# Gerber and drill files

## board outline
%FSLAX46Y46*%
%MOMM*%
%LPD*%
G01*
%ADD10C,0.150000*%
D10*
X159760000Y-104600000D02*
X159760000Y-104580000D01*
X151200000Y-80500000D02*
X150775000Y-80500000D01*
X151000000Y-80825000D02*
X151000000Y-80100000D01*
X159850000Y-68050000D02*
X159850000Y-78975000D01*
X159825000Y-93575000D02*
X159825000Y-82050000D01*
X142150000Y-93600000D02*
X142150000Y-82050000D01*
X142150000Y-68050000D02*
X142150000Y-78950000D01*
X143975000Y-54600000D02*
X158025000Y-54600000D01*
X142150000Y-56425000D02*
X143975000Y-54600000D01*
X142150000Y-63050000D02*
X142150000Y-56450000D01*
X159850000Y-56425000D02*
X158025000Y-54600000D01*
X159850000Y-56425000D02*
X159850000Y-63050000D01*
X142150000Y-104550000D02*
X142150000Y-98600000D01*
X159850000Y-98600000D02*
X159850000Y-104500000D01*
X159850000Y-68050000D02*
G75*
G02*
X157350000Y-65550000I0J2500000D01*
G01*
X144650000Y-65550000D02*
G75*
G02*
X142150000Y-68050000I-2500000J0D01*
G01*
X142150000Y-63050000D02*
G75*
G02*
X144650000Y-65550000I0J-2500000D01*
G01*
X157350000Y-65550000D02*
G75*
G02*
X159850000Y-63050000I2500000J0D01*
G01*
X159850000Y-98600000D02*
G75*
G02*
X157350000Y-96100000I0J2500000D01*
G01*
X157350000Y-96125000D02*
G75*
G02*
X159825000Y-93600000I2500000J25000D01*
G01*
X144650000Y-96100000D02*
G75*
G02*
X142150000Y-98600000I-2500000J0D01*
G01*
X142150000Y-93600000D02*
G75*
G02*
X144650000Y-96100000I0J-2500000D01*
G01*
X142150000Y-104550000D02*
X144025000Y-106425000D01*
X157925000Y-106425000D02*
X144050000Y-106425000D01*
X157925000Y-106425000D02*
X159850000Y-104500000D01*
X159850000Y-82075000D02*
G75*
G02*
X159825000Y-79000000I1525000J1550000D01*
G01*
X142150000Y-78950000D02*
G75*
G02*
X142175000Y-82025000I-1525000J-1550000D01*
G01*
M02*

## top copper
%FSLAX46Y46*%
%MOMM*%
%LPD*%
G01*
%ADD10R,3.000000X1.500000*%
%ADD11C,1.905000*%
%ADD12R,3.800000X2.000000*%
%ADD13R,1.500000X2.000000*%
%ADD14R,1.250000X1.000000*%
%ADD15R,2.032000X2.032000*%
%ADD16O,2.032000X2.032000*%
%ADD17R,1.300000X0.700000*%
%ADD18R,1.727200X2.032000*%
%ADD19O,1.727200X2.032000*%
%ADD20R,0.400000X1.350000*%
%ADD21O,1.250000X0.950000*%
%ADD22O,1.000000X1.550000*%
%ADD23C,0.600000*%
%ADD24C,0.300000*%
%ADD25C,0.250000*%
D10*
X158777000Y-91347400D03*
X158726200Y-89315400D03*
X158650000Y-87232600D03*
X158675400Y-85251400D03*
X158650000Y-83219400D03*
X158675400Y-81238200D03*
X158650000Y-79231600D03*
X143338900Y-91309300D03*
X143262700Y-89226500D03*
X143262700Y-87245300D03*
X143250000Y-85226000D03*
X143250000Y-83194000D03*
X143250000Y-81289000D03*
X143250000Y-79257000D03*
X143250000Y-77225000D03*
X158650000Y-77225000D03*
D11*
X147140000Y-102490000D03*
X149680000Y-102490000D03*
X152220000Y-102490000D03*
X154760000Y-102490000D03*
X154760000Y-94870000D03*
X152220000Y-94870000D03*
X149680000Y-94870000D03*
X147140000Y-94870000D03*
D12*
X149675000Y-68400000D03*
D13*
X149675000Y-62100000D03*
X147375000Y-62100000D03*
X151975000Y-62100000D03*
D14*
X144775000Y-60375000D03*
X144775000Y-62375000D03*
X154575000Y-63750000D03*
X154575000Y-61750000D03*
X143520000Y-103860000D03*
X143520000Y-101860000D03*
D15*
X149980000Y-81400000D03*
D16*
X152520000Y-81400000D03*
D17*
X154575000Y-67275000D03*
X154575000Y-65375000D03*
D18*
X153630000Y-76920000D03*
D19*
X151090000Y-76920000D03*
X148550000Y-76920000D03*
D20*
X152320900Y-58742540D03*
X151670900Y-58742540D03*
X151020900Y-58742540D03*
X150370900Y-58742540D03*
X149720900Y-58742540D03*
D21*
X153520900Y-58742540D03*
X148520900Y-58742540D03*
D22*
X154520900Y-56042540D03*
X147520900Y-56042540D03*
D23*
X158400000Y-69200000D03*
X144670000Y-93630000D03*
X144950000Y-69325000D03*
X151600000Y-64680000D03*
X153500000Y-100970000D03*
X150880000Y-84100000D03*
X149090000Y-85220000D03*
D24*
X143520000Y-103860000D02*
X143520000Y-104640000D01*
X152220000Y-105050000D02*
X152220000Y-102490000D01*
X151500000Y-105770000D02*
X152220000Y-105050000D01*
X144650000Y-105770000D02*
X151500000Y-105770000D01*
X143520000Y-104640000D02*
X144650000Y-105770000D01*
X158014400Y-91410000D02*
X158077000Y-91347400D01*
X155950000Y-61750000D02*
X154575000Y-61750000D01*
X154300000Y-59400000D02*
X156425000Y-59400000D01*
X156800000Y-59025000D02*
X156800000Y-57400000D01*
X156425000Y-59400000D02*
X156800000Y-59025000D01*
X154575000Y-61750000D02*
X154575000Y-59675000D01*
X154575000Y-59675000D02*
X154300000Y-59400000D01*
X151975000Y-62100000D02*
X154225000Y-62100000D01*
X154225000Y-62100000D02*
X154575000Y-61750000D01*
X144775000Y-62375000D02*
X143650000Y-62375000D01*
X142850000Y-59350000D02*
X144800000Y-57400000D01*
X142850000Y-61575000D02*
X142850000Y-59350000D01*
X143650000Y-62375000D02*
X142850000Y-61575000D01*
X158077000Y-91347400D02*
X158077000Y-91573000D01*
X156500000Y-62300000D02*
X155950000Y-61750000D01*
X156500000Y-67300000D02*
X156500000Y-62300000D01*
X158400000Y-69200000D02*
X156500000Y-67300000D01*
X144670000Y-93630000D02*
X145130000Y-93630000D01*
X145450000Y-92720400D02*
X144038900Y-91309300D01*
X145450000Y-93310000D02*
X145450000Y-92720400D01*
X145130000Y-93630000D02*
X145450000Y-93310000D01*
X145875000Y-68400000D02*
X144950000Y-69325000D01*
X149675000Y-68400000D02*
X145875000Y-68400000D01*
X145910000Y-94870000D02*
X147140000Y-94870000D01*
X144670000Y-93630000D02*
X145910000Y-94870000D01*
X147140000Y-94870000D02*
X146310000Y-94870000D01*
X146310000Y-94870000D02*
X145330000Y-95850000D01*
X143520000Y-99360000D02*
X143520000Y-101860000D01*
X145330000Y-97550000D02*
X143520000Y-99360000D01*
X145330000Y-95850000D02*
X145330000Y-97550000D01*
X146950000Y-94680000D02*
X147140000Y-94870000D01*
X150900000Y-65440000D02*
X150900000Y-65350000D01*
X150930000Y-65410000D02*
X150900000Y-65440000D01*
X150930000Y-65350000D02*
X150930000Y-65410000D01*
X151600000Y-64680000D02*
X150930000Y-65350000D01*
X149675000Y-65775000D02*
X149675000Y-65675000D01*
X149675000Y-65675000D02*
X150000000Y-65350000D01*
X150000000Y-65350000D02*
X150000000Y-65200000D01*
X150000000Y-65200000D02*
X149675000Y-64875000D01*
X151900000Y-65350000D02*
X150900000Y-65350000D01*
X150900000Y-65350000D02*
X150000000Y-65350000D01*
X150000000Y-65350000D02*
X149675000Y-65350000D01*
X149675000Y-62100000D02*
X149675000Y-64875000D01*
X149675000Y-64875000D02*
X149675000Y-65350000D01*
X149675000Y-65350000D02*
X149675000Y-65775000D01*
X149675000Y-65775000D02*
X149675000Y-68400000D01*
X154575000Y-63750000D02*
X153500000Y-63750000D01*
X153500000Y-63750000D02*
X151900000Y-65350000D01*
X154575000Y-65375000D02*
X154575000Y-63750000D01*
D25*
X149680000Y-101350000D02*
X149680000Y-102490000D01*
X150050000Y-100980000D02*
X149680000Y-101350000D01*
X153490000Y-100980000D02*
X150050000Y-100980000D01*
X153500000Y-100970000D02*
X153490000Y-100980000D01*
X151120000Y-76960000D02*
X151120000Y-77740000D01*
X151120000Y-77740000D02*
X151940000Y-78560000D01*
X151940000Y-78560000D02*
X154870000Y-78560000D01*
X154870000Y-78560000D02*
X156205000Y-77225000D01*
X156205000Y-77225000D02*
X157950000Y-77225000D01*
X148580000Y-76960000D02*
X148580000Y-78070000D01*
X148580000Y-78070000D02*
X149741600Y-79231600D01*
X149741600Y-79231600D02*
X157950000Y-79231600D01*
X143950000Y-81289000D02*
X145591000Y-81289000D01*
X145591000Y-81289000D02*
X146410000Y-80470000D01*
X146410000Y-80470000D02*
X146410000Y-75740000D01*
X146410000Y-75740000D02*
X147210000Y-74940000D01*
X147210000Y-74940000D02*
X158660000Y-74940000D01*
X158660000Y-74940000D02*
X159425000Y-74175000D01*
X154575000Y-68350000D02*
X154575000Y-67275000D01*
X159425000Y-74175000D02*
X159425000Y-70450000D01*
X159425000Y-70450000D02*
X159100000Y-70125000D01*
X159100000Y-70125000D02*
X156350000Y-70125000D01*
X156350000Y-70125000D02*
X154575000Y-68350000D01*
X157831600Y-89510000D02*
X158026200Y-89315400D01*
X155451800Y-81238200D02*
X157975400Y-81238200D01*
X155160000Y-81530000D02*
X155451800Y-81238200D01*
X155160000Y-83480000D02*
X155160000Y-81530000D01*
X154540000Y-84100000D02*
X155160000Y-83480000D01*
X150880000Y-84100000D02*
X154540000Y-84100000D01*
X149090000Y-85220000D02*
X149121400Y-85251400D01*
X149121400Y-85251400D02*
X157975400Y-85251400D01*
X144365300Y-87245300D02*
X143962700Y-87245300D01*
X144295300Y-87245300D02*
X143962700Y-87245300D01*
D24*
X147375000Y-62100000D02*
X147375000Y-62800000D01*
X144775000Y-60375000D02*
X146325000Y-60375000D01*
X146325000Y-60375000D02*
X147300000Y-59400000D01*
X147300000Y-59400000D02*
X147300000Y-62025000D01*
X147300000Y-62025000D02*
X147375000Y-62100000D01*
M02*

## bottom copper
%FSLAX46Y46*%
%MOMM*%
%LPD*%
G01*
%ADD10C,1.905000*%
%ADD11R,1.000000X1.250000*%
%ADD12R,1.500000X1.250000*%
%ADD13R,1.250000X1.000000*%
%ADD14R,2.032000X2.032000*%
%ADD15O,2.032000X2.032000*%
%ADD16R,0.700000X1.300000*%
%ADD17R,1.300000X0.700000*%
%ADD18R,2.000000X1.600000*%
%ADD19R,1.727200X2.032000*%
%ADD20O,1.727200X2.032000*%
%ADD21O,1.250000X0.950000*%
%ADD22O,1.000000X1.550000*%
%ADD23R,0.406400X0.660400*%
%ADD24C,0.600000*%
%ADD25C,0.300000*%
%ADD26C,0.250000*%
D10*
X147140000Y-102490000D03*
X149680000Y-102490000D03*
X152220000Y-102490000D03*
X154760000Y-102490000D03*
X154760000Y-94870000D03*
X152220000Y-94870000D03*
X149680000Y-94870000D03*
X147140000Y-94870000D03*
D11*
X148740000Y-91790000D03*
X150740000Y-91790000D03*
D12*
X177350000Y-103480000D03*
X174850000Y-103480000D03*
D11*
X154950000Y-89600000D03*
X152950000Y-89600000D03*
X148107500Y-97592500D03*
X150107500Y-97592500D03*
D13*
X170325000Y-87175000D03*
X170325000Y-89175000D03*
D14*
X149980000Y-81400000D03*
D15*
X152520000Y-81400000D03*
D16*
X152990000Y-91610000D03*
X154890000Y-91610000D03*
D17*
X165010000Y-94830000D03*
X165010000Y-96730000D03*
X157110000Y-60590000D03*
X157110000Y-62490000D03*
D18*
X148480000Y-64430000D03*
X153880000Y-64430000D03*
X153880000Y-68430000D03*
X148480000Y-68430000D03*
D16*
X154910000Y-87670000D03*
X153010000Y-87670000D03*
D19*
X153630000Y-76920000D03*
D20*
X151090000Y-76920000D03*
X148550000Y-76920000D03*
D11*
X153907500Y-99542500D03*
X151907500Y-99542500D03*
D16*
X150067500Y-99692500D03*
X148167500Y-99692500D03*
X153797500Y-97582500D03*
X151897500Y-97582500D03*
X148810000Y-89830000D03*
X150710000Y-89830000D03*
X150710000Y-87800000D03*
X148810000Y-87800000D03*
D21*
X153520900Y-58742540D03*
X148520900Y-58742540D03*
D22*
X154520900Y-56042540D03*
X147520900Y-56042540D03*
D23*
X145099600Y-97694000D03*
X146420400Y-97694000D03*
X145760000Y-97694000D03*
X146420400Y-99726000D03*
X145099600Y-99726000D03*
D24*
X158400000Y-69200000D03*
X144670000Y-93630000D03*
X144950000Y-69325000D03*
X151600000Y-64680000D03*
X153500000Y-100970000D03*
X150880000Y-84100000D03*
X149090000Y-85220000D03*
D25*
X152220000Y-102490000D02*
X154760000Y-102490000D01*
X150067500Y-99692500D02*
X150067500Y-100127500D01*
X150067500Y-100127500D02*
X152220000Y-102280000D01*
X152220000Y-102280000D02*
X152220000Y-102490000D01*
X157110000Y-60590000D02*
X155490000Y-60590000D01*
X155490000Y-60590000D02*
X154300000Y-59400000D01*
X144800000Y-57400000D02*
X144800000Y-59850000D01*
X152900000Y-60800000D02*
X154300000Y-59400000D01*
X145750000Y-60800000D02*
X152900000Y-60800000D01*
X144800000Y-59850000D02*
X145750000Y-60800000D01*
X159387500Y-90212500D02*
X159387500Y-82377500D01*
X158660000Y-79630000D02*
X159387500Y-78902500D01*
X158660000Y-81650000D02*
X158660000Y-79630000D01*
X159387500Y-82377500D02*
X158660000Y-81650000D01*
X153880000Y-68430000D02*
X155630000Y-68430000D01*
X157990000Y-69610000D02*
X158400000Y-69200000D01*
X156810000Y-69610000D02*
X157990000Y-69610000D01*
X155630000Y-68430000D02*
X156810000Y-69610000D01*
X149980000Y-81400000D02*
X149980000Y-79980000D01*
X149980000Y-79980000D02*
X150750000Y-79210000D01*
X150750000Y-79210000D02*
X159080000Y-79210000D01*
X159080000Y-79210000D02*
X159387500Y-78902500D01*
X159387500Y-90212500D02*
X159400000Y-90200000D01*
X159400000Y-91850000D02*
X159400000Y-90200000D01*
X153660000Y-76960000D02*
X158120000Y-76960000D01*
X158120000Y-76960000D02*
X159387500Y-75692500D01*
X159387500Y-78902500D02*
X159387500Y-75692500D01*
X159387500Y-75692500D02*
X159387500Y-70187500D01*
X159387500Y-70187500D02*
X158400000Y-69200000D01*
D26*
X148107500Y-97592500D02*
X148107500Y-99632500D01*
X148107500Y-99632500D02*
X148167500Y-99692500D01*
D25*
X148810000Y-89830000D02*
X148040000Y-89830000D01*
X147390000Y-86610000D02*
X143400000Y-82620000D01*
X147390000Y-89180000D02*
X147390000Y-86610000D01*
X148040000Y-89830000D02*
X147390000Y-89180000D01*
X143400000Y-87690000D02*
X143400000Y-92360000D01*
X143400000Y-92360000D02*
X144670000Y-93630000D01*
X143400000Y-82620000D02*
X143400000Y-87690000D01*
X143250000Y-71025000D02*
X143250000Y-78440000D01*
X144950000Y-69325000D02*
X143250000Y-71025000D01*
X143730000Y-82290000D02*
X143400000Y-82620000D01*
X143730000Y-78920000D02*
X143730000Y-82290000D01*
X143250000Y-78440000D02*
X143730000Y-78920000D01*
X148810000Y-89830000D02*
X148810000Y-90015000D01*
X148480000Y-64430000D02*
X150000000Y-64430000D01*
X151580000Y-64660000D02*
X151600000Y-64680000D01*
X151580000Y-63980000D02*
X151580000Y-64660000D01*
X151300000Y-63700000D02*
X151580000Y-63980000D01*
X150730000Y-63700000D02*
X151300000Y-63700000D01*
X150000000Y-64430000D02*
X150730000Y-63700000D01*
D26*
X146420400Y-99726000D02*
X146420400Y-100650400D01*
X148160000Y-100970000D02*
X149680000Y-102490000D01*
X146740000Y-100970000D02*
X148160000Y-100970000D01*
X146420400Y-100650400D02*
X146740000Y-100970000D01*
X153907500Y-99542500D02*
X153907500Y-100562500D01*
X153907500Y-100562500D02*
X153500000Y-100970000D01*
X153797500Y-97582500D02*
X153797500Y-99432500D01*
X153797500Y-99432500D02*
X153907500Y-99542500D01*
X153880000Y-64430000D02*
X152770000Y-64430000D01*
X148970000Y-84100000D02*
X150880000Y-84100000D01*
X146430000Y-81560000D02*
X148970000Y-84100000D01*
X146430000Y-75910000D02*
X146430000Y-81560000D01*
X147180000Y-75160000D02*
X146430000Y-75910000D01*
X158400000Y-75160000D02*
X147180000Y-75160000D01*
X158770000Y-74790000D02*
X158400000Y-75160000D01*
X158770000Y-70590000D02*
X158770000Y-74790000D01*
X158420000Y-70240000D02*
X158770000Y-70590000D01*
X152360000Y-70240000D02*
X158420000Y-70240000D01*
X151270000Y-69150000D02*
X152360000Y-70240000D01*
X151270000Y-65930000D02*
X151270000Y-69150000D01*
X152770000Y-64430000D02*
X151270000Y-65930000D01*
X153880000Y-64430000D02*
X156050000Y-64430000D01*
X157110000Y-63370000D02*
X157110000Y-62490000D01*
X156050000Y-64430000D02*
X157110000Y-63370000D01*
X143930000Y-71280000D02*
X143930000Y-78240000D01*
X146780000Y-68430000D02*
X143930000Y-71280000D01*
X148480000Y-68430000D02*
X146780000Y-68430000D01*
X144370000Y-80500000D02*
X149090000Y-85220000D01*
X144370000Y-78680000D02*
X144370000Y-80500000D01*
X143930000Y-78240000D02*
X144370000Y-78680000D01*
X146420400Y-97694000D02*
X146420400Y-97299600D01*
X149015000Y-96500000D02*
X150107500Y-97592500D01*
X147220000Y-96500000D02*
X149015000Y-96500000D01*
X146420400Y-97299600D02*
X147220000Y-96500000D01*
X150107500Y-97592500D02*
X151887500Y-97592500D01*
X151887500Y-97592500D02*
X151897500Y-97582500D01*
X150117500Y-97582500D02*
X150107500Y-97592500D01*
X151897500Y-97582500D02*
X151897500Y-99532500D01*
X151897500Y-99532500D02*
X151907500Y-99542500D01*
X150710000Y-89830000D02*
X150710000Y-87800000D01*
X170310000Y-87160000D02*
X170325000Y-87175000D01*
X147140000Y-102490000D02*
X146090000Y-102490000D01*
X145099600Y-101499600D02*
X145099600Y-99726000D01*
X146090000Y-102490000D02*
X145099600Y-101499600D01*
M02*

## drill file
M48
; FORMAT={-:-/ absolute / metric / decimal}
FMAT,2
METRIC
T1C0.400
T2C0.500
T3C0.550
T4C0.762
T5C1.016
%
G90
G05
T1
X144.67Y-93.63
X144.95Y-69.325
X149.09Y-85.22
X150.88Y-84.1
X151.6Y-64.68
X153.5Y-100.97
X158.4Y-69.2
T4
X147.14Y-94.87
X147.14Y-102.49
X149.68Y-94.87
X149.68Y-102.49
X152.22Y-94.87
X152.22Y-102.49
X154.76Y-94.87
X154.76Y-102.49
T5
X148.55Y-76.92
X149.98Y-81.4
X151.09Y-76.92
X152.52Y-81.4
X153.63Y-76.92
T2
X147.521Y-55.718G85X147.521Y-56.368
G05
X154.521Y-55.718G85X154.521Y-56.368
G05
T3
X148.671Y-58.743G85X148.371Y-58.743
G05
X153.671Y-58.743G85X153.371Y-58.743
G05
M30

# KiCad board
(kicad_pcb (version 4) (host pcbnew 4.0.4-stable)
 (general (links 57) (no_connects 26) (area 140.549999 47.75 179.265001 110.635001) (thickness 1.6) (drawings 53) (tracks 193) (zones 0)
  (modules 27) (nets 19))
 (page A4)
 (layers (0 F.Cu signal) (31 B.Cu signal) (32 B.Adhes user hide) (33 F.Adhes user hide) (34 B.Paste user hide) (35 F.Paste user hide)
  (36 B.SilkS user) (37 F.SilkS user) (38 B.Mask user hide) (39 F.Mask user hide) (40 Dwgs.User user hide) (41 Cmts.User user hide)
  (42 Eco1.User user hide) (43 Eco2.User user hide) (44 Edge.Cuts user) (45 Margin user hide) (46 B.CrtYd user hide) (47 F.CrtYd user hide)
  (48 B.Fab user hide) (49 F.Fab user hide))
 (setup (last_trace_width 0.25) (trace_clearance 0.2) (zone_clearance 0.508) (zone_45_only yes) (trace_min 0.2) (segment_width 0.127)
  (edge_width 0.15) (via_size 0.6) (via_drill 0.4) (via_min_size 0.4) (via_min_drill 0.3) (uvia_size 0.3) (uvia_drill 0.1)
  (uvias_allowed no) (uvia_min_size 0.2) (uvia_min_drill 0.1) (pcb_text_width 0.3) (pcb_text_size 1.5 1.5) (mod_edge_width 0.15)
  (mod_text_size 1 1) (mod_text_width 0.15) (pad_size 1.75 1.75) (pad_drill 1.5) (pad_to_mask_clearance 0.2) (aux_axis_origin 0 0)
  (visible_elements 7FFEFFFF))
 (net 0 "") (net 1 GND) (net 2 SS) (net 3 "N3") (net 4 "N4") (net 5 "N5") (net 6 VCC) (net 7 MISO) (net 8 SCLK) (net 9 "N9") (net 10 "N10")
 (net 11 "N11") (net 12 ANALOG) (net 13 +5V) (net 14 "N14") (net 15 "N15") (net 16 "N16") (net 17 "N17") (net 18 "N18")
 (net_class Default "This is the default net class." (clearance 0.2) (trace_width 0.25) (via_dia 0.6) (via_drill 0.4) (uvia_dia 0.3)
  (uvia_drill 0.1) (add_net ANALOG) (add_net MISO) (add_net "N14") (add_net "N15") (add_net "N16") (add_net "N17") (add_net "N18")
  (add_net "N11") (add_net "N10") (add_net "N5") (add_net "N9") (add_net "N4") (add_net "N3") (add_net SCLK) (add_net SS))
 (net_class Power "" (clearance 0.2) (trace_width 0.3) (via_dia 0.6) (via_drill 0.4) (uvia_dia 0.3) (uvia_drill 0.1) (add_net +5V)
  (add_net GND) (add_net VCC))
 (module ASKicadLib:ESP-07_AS (layer F.Cu) (at 143.95 77.225)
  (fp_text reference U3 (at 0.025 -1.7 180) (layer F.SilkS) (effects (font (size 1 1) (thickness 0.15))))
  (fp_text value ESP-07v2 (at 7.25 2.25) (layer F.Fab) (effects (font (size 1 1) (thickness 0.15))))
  (pad 9 smd rect (at 14.127 14.1224) (size 3 1.5) (drill (offset 0.7 0)) (layers F.Cu F.Paste F.Mask) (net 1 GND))
  (pad 10 smd rect (at 14.0762 12.0904) (size 3 1.5) (drill (offset 0.7 0)) (layers F.Cu F.Paste F.Mask) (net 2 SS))
  (pad 11 smd rect (at 14 10.0076) (size 3 1.5) (drill (offset 0.7 0)) (layers F.Cu F.Paste F.Mask))
  (pad 12 smd rect (at 14.0254 8.0264) (size 3 1.5) (drill (offset 0.7 0)) (layers F.Cu F.Paste F.Mask) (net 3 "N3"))
  (pad 13 smd rect (at 14 5.9944) (size 3 1.5) (drill (offset 0.7 0)) (layers F.Cu F.Paste F.Mask))
  (pad 14 smd rect (at 14.0254 4.0132) (size 3 1.5) (drill (offset 0.7 0)) (layers F.Cu F.Paste F.Mask) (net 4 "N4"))
  (pad 15 smd rect (at 14 2.0066) (size 3 1.5) (drill (offset 0.7 0)) (layers F.Cu F.Paste F.Mask) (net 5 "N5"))
  (pad 8 smd rect (at 0.0889 14.0843) (size 3 1.5) (drill (offset -0.7 0)) (layers F.Cu F.Paste F.Mask) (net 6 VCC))
  (pad 7 smd rect (at 0.0127 12.0015) (size 3 1.5) (drill (offset -0.7 0)) (layers F.Cu F.Paste F.Mask))
  (pad 6 smd rect (at 0.0127 10.0203) (size 3 1.5) (drill (offset -0.7 0)) (layers F.Cu F.Paste F.Mask) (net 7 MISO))
  (pad 5 smd rect (at 0 8.001) (size 3 1.5) (drill (offset -0.7 0)) (layers F.Cu F.Paste F.Mask) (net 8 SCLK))
  (pad 4 smd rect (at 0 5.969) (size 3 1.5) (drill (offset -0.7 0)) (layers F.Cu F.Paste F.Mask))
  (pad 3 smd rect (at 0 4.064) (size 3 1.5) (drill (offset -0.7 0)) (layers F.Cu F.Paste F.Mask) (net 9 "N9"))
  (pad 2 smd rect (at 0 2.032) (size 3 1.5) (drill (offset -0.7 0)) (layers F.Cu F.Paste F.Mask))
  (pad 1 smd rect (at 0 0) (size 3 1.5) (drill (offset -0.7 0)) (layers F.Cu F.Paste F.Mask))
  (pad 16 smd rect (at 14 0) (size 3 1.5) (drill (offset 0.7 0)) (layers F.Cu F.Paste F.Mask) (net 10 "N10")))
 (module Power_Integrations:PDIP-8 (layer F.Cu) (at 150.95 98.68)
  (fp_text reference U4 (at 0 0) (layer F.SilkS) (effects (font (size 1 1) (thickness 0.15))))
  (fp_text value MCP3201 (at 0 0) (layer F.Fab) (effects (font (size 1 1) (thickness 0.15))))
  (pad 1 thru_hole circle (at -3.81 3.81) (size 1.905 1.905) (drill 0.762) (layers *.Cu *.Mask) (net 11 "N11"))
  (pad 2 thru_hole circle (at -1.27 3.81) (size 1.905 1.905) (drill 0.762) (layers *.Cu *.Mask) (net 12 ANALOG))
  (pad 3 thru_hole circle (at 1.27 3.81) (size 1.905 1.905) (drill 0.762) (layers *.Cu *.Mask) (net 1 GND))
  (pad 4 thru_hole circle (at 3.81 3.81) (size 1.905 1.905) (drill 0.762) (layers *.Cu *.Mask) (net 1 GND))
  (pad 5 thru_hole circle (at 3.81 -3.81) (size 1.905 1.905) (drill 0.762) (layers *.Cu *.Mask) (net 2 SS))
  (pad 6 thru_hole circle (at 1.27 -3.81) (size 1.905 1.905) (drill 0.762) (layers *.Cu *.Mask) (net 7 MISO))
  (pad 7 thru_hole circle (at -1.27 -3.81) (size 1.905 1.905) (drill 0.762) (layers *.Cu *.Mask) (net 8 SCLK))
  (pad 8 thru_hole circle (at -3.81 -3.81) (size 1.905 1.905) (drill 0.762) (layers *.Cu *.Mask) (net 6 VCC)))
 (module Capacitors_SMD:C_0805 (layer B.Cu) (at 149.74 91.79)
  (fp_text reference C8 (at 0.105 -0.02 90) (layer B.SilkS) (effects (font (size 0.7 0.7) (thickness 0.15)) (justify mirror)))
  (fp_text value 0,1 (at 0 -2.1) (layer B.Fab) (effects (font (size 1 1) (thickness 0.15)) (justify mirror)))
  (pad 1 smd rect (at -1 0) (size 1 1.25) (layers B.Cu B.Paste B.Mask) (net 1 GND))
  (pad 2 smd rect (at 1 0) (size 1 1.25) (layers B.Cu B.Paste B.Mask) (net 11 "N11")))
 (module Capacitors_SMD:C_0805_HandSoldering (layer B.Cu) (at 176.1 103.48 180)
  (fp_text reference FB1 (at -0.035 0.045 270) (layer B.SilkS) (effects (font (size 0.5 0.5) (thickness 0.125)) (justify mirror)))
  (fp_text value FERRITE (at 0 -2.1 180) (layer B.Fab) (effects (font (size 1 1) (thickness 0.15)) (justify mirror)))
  (pad 1 smd rect (at -1.25 0 180) (size 1.5 1.25) (layers B.Cu B.Paste B.Mask) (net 11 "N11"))
  (pad 2 smd rect (at 1.25 0 180) (size 1.5 1.25) (layers B.Cu B.Paste B.Mask) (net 6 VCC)))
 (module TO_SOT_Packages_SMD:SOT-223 (layer F.Cu) (at 149.675 65.25 270)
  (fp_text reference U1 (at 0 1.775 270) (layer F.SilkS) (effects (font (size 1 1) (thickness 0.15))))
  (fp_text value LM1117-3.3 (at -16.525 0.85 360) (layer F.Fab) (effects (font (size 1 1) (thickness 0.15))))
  (pad 4 smd rect (at 3.15 0 270) (size 2 3.8) (layers F.Cu F.Paste F.Mask) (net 6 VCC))
  (pad 2 smd rect (at -3.15 0 270) (size 2 1.5) (layers F.Cu F.Paste F.Mask) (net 6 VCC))
  (pad 3 smd rect (at -3.15 2.3 270) (size 2 1.5) (layers F.Cu F.Paste F.Mask) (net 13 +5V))
  (pad 1 smd rect (at -3.15 -2.3 270) (size 2 1.5) (layers F.Cu F.Paste F.Mask) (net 1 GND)))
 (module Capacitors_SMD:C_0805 (layer F.Cu) (at 144.775 61.375 270)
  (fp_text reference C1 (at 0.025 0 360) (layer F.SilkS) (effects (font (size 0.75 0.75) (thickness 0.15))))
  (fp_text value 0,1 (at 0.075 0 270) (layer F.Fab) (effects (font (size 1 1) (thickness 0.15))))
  (pad 1 smd rect (at -1 0 270) (size 1 1.25) (layers F.Cu F.Paste F.Mask) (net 13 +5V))
  (pad 2 smd rect (at 1 0 270) (size 1 1.25) (layers F.Cu F.Paste F.Mask) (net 1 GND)))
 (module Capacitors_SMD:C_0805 (layer B.Cu) (at 153.95 89.6 180)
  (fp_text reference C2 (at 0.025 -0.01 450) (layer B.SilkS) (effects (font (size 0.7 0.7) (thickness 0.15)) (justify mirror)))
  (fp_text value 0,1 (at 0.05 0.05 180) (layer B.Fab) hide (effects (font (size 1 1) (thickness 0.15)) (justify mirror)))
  (pad 1 smd rect (at -1 0 180) (size 1 1.25) (layers B.Cu B.Paste B.Mask) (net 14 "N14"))
  (pad 2 smd rect (at 1 0 180) (size 1 1.25) (layers B.Cu B.Paste B.Mask) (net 1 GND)))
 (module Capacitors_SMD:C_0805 (layer B.Cu) (at 149.1075 97.5925)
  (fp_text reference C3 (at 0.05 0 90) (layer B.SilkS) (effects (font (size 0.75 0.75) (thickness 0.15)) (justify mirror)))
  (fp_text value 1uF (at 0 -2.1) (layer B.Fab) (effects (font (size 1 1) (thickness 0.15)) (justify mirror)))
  (pad 1 smd rect (at -1 0) (size 1 1.25) (layers B.Cu B.Paste B.Mask) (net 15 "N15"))
  (pad 2 smd rect (at 1 0) (size 1 1.25) (layers B.Cu B.Paste B.Mask) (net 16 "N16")))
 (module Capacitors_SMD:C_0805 (layer F.Cu) (at 154.575 62.75 90)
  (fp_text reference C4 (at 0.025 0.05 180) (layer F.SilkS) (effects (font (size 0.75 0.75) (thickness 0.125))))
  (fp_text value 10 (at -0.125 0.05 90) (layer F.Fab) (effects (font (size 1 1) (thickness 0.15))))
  (pad 1 smd rect (at -1 0 90) (size 1 1.25) (layers F.Cu F.Paste F.Mask) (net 6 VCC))
  (pad 2 smd rect (at 1 0 90) (size 1 1.25) (layers F.Cu F.Paste F.Mask) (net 1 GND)))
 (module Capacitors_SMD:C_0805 (layer B.Cu) (at 170.325 88.175 270)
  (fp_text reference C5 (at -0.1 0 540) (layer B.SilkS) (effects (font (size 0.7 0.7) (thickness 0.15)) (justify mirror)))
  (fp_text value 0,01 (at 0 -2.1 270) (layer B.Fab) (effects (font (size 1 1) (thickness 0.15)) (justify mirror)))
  (pad 1 smd rect (at -1 0 270) (size 1 1.25) (layers B.Cu B.Paste B.Mask) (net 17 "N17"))
  (pad 2 smd rect (at 1 0 270) (size 1 1.25) (layers B.Cu B.Paste B.Mask) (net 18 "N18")))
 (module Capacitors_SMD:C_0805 (layer F.Cu) (at 143.52 102.86 90)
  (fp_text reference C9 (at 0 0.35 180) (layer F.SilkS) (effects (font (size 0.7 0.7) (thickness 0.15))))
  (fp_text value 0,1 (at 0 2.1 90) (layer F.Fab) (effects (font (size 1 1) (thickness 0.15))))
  (pad 1 smd rect (at -1 0 90) (size 1 1.25) (layers F.Cu F.Paste F.Mask) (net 1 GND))
  (pad 2 smd rect (at 1 0 90) (size 1 1.25) (layers F.Cu F.Paste F.Mask) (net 6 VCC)))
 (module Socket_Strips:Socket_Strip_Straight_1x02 (layer F.Cu) (at 149.98 81.4)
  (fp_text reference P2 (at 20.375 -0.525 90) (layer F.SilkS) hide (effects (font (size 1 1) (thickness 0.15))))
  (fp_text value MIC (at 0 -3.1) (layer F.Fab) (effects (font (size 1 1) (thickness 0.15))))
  (pad 1 thru_hole rect (at 0 0) (size 2.032 2.032) (drill 1.016) (layers *.Cu *.Mask) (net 1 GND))
  (pad 2 thru_hole oval (at 2.54 0) (size 2.032 2.032) (drill 1.016) (layers *.Cu *.Mask) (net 18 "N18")))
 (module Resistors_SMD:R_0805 (layer B.Cu) (at 153.94 91.61)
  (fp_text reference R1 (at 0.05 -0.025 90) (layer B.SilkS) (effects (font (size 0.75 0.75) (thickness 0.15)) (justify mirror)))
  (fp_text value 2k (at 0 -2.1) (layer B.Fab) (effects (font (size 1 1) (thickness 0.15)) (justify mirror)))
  (pad 1 smd rect (at -0.95 0) (size 0.7 1.3) (layers B.Cu B.Paste B.Mask) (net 6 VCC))
  (pad 2 smd rect (at 0.95 0) (size 0.7 1.3) (layers B.Cu B.Paste B.Mask) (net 14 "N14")))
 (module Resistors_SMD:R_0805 (layer F.Cu) (at 154.575 66.325 90)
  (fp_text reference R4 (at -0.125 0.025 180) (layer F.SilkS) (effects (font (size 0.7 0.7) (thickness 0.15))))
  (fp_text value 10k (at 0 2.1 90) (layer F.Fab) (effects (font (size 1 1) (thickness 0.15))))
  (pad 1 smd rect (at -0.95 0 90) (size 0.7 1.3) (layers F.Cu F.Paste F.Mask) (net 9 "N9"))
  (pad 2 smd rect (at 0.95 0 90) (size 0.7 1.3) (layers F.Cu F.Paste F.Mask) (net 6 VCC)))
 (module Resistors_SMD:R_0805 (layer B.Cu) (at 165.01 95.78 270)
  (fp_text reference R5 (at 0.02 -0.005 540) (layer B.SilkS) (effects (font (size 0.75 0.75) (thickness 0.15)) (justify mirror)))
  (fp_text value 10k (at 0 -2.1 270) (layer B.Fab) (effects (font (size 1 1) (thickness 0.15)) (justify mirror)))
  (pad 1 smd rect (at -0.95 0 270) (size 0.7 1.3) (layers B.Cu B.Paste B.Mask) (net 2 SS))
  (pad 2 smd rect (at 0.95 0 270) (size 0.7 1.3) (layers B.Cu B.Paste B.Mask) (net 1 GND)))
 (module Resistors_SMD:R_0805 (layer B.Cu) (at 157.11 61.54 270)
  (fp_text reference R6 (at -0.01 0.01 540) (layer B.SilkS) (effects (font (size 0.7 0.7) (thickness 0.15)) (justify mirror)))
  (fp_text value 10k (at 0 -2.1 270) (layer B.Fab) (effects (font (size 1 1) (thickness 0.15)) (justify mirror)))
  (pad 1 smd rect (at -0.95 0 270) (size 0.7 1.3) (layers B.Cu B.Paste B.Mask) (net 1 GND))
  (pad 2 smd rect (at 0.95 0 270) (size 0.7 1.3) (layers B.Cu B.Paste B.Mask) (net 4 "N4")))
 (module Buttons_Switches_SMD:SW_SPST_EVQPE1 (layer B.Cu) (at 151.18 64.43 180)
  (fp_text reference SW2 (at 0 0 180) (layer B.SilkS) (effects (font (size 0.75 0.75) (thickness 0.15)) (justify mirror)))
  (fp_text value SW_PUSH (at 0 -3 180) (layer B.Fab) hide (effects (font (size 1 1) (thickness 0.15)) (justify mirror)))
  (pad 2 smd rect (at 2.7 0 180) (size 2 1.6) (layers B.Cu B.Paste B.Mask) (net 6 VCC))
  (pad 1 smd rect (at -2.7 0 180) (size 2 1.6) (layers B.Cu B.Paste B.Mask) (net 4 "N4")))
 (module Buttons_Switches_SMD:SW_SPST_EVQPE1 (layer B.Cu) (at 151.18 68.43)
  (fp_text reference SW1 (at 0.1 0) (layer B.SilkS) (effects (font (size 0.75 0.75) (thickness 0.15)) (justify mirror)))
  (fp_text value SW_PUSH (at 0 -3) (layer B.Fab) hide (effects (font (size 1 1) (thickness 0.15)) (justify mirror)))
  (pad 2 smd rect (at 2.7 0) (size 2 1.6) (layers B.Cu B.Paste B.Mask) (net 1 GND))
  (pad 1 smd rect (at -2.7 0) (size 2 1.6) (layers B.Cu B.Paste B.Mask) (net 3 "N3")))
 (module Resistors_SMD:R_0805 (layer B.Cu) (at 153.96 87.67 180)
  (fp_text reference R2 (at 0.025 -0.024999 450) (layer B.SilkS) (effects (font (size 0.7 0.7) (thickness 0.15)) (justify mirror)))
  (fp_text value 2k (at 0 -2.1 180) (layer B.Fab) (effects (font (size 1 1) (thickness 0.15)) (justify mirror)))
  (pad 1 smd rect (at -0.95 0 180) (size 0.7 1.3) (layers B.Cu B.Paste B.Mask) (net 14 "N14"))
  (pad 2 smd rect (at 0.95 0 180) (size 0.7 1.3) (layers B.Cu B.Paste B.Mask) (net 18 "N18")))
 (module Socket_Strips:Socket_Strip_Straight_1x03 (layer F.Cu) (at 153.63 76.92 180)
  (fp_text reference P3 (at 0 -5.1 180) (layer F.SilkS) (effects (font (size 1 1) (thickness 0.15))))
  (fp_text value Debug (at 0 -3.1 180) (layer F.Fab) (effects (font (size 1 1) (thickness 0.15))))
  (pad 1 thru_hole rect (at 0 0 180) (size 1.7272 2.032) (drill 1.016) (layers *.Cu *.Mask) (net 1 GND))
  (pad 2 thru_hole oval (at 2.54 0 180) (size 1.7272 2.032) (drill 1.016) (layers *.Cu *.Mask) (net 10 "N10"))
  (pad 3 thru_hole oval (at 5.08 0 180) (size 1.7272 2.032) (drill 1.016) (layers *.Cu *.Mask) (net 5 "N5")))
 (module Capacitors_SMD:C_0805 (layer B.Cu) (at 152.9075 99.5425 180)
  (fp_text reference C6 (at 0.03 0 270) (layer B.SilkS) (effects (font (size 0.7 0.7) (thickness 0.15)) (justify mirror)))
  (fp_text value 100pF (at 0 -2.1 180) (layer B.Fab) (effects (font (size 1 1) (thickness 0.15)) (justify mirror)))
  (pad 1 smd rect (at -1 0 180) (size 1 1.25) (layers B.Cu B.Paste B.Mask) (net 12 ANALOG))
  (pad 2 smd rect (at 1 0 180) (size 1 1.25) (layers B.Cu B.Paste B.Mask) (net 16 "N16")))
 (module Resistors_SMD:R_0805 (layer B.Cu) (at 149.1175 99.6925 180)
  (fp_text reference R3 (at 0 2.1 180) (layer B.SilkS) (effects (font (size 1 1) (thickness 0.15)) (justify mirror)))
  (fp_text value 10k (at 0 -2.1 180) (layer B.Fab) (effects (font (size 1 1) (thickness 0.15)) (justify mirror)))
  (pad 1 smd rect (at -0.95 0 180) (size 0.7 1.3) (layers B.Cu B.Paste B.Mask) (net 1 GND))
  (pad 2 smd rect (at 0.95 0 180) (size 0.7 1.3) (layers B.Cu B.Paste B.Mask) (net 15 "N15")))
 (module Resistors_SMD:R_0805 (layer B.Cu) (at 152.8475 97.5825 180)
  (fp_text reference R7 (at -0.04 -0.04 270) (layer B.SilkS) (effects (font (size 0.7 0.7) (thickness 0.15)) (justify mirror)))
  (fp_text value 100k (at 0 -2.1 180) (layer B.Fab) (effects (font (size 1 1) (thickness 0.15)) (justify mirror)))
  (pad 1 smd rect (at -0.95 0 180) (size 0.7 1.3) (layers B.Cu B.Paste B.Mask) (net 12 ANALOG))
  (pad 2 smd rect (at 0.95 0 180) (size 0.7 1.3) (layers B.Cu B.Paste B.Mask) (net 16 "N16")))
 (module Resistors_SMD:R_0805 (layer B.Cu) (at 149.76 89.83)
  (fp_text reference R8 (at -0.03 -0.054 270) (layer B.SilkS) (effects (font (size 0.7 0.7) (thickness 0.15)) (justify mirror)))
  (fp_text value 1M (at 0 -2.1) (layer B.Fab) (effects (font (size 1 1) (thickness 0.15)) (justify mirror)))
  (pad 1 smd rect (at -0.95 0) (size 0.7 1.3) (layers B.Cu B.Paste B.Mask) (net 6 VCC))
  (pad 2 smd rect (at 0.95 0) (size 0.7 1.3) (layers B.Cu B.Paste B.Mask) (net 17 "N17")))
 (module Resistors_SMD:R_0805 (layer B.Cu) (at 149.76 87.8 180)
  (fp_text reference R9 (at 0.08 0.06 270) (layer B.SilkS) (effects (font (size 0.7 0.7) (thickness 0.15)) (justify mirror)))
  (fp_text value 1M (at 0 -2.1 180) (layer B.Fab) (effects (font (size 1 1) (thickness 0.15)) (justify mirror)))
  (pad 1 smd rect (at -0.95 0 180) (size 0.7 1.3) (layers B.Cu B.Paste B.Mask) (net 17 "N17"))
  (pad 2 smd rect (at 0.95 0 180) (size 0.7 1.3) (layers B.Cu B.Paste B.Mask) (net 1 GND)))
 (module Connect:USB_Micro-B (layer F.Cu) (at 151.02 57.18 180)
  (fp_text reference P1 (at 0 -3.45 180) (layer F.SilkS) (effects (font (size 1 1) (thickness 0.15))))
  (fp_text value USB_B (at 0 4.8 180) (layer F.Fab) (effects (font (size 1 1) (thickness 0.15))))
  (pad 1 smd rect (at -1.3009 -1.56254 270) (size 1.35 0.4) (layers F.Cu F.Paste F.Mask) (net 13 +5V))
  (pad 2 smd rect (at -0.6509 -1.56254 270) (size 1.35 0.4) (layers F.Cu F.Paste F.Mask))
  (pad 3 smd rect (at -0.0009 -1.56254 270) (size 1.35 0.4) (layers F.Cu F.Paste F.Mask))
  (pad 4 smd rect (at 0.6491 -1.56254 270) (size 1.35 0.4) (layers F.Cu F.Paste F.Mask) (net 1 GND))
  (pad 5 smd rect (at 1.2991 -1.56254 270) (size 1.35 0.4) (layers F.Cu F.Paste F.Mask) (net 1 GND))
  (pad 6 thru_hole oval (at -2.5009 -1.56254 270) (size 0.95 1.25) (drill oval 0.55 0.85) (layers *.Cu *.Mask))
  (pad 6 thru_hole oval (at 2.4991 -1.56254 270) (size 0.95 1.25) (drill oval 0.55 0.85) (layers *.Cu *.Mask))
  (pad 6 thru_hole oval (at -3.5009 1.13746 270) (size 1.55 1) (drill oval 1.15 0.5) (layers *.Cu *.Mask))
  (pad 6 thru_hole oval (at 3.4991 1.13746 270) (size 1.55 1) (drill oval 1.15 0.5) (layers *.Cu *.Mask)))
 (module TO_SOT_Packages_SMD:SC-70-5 (layer B.Cu) (at 145.76 98.71)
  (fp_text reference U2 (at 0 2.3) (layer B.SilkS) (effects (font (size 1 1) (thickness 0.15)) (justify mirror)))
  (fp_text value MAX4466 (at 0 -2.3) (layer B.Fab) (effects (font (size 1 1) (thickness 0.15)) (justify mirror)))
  (pad 1 smd rect (at -0.6604 -1.016) (size 0.4064 0.6604) (layers B.Cu B.Paste B.Mask) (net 17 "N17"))
  (pad 3 smd rect (at 0.6604 -1.016) (size 0.4064 0.6604) (layers B.Cu B.Paste B.Mask) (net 16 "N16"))
  (pad 2 smd rect (at 0 -1.016) (size 0.4064 0.6604) (layers B.Cu B.Paste B.Mask) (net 1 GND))
  (pad 4 smd rect (at 0.6604 1.016) (size 0.4064 0.6604) (layers B.Cu B.Paste B.Mask) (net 12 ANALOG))
  (pad 5 smd rect (at -0.6604 1.016) (size 0.4064 0.6604) (layers B.Cu B.Paste B.Mask) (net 11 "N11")))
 (gr_line (start 159.76 104.6) (end 159.76 104.58) (angle 90) (layer Edge.Cuts) (width 0.15))
 (gr_line (start 151.2 80.5) (end 150.775 80.5) (angle 90) (layer Edge.Cuts) (width 0.15))
 (gr_line (start 151 80.825) (end 151 80.1) (angle 90) (layer Edge.Cuts) (width 0.15))
 (gr_line (start 159.85 68.05) (end 159.85 78.975) (angle 90) (layer Edge.Cuts) (width 0.15))
 (gr_line (start 159.825 93.575) (end 159.825 82.05) (angle 90) (layer Edge.Cuts) (width 0.15))
 (gr_line (start 142.15 93.6) (end 142.15 82.05) (angle 90) (layer Edge.Cuts) (width 0.15))
 (gr_line (start 142.15 68.05) (end 142.15 78.95) (angle 90) (layer Edge.Cuts) (width 0.15))
 (gr_line (start 143.975 54.6) (end 158.025 54.6) (angle 90) (layer Edge.Cuts) (width 0.15))
 (gr_line (start 142.15 56.425) (end 143.975 54.6) (angle 90) (layer Edge.Cuts) (width 0.15))
 (gr_line (start 142.15 63.05) (end 142.15 56.45) (angle 90) (layer Edge.Cuts) (width 0.15))
 (gr_line (start 159.85 56.425) (end 158.025 54.6) (angle 90) (layer Edge.Cuts) (width 0.15))
 (gr_line (start 159.85 56.425) (end 159.85 63.05) (angle 90) (layer Edge.Cuts) (width 0.15))
 (gr_line (start 142.15 104.55) (end 142.15 98.6) (angle 90) (layer Edge.Cuts) (width 0.15))
 (gr_line (start 159.85 98.6) (end 159.85 104.5) (angle 90) (layer Edge.Cuts) (width 0.15))
 (gr_arc (start 159.85 65.55) (end 159.85 68.05) (angle 90) (layer Edge.Cuts) (width 0.15))
 (gr_arc (start 142.15 65.55) (end 144.65 65.55) (angle 90) (layer Edge.Cuts) (width 0.15))
 (gr_arc (start 142.15 65.55) (end 142.15 63.05) (angle 90) (layer Edge.Cuts) (width 0.15))
 (gr_arc (start 159.85 65.55) (end 157.35 65.55) (angle 90) (layer Edge.Cuts) (width 0.15))
 (gr_arc (start 159.85 96.1) (end 159.85 98.6) (angle 90) (layer Edge.Cuts) (width 0.15))
 (gr_arc (start 159.85 96.1) (end 157.35 96.125) (angle 90) (layer Edge.Cuts) (width 0.15))
 (gr_arc (start 142.15 96.1) (end 144.65 96.1) (angle 90) (layer Edge.Cuts) (width 0.15))
 (gr_arc (start 142.15 96.1) (end 142.15 93.6) (angle 90) (layer Edge.Cuts) (width 0.15))
 (gr_line (start 142.15 104.55) (end 144.025 106.425) (angle 90) (layer Edge.Cuts) (width 0.15))
 (gr_line (start 157.925 106.425) (end 144.05 106.425) (angle 90) (layer Edge.Cuts) (width 0.15))
 (gr_line (start 157.925 106.425) (end 159.85 104.5) (angle 90) (layer Edge.Cuts) (width 0.15))
 (gr_arc (start 161.375 80.525) (end 159.85 82.075) (angle 90) (layer Edge.Cuts) (width 0.15))
 (gr_arc (start 140.625 80.5) (end 142.15 78.95) (angle 90) (layer Edge.Cuts) (width 0.15))
 (segment (start 143.52 103.86) (end 143.52 104.64) (width 0.3) (layer F.Cu) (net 1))
 (segment (start 152.22 105.05) (end 152.22 102.49) (width 0.3) (layer F.Cu) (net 1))
 (segment (start 151.5 105.77) (end 152.22 105.05) (width 0.3) (layer F.Cu) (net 1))
 (segment (start 144.65 105.77) (end 151.5 105.77) (width 0.3) (layer F.Cu) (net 1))
 (segment (start 143.52 104.64) (end 144.65 105.77) (width 0.3) (layer F.Cu) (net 1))
 (segment (start 152.22 102.49) (end 154.76 102.49) (width 0.3) (layer B.Cu) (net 1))
 (segment (start 150.0675 99.6925) (end 150.0675 100.1275) (width 0.3) (layer B.Cu) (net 1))
 (segment (start 150.0675 100.1275) (end 152.22 102.28) (width 0.3) (layer B.Cu) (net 1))
 (segment (start 152.22 102.28) (end 152.22 102.49) (width 0.3) (layer B.Cu) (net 1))
 (segment (start 157.11 60.59) (end 155.49 60.59) (width 0.3) (layer B.Cu) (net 1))
 (segment (start 155.49 60.59) (end 154.3 59.4) (width 0.3) (layer B.Cu) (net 1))
 (segment (start 144.8 57.4) (end 144.8 59.85) (width 0.3) (layer B.Cu) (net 1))
 (segment (start 152.9 60.8) (end 154.3 59.4) (width 0.3) (layer B.Cu) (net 1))
 (segment (start 145.75 60.8) (end 152.9 60.8) (width 0.3) (layer B.Cu) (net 1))
 (segment (start 144.8 59.85) (end 145.75 60.8) (width 0.3) (layer B.Cu) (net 1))
 (segment (start 159.3875 90.2125) (end 159.3875 82.3775) (width 0.3) (layer B.Cu) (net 1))
 (segment (start 158.66 79.63) (end 159.3875 78.9025) (width 0.3) (layer B.Cu) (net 1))
 (segment (start 158.66 81.65) (end 158.66 79.63) (width 0.3) (layer B.Cu) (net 1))
 (segment (start 159.3875 82.3775) (end 158.66 81.65) (width 0.3) (layer B.Cu) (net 1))
 (segment (start 153.88 68.43) (end 155.63 68.43) (width 0.3) (layer B.Cu) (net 1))
 (segment (start 157.99 69.61) (end 158.4 69.2) (width 0.3) (layer B.Cu) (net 1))
 (segment (start 156.81 69.61) (end 157.99 69.61) (width 0.3) (layer B.Cu) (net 1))
 (segment (start 155.63 68.43) (end 156.81 69.61) (width 0.3) (layer B.Cu) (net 1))
 (segment (start 149.98 81.4) (end 149.98 79.98) (width 0.3) (layer B.Cu) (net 1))
 (segment (start 149.98 79.98) (end 150.75 79.21) (width 0.3) (layer B.Cu) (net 1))
 (segment (start 150.75 79.21) (end 159.08 79.21) (width 0.3) (layer B.Cu) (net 1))
 (segment (start 159.08 79.21) (end 159.3875 78.9025) (width 0.3) (layer B.Cu) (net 1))
 (segment (start 158.0144 91.41) (end 158.077 91.3474) (width 0.3) (layer F.Cu) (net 1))
 (segment (start 155.95 61.75) (end 154.575 61.75) (width 0.3) (layer F.Cu) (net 1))
 (segment (start 154.3 59.4) (end 156.425 59.4) (width 0.3) (layer F.Cu) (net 1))
 (segment (start 156.8 59.025) (end 156.8 57.4) (width 0.3) (layer F.Cu) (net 1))
 (segment (start 156.425 59.4) (end 156.8 59.025) (width 0.3) (layer F.Cu) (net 1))
 (segment (start 154.575 61.75) (end 154.575 59.675) (width 0.3) (layer F.Cu) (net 1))
 (segment (start 154.575 59.675) (end 154.3 59.4) (width 0.3) (layer F.Cu) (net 1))
 (segment (start 151.975 62.1) (end 154.225 62.1) (width 0.3) (layer F.Cu) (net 1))
 (segment (start 154.225 62.1) (end 154.575 61.75) (width 0.3) (layer F.Cu) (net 1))
 (segment (start 144.775 62.375) (end 143.65 62.375) (width 0.3) (layer F.Cu) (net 1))
 (segment (start 142.85 59.35) (end 144.8 57.4) (width 0.3) (layer F.Cu) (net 1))
 (segment (start 142.85 61.575) (end 142.85 59.35) (width 0.3) (layer F.Cu) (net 1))
 (segment (start 143.65 62.375) (end 142.85 61.575) (width 0.3) (layer F.Cu) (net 1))
 (segment (start 159.3875 90.2125) (end 159.4 90.2) (width 0.3) (layer B.Cu) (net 1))
 (segment (start 159.4 91.85) (end 159.4 90.2) (width 0.3) (layer B.Cu) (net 1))
 (segment (start 158.077 91.3474) (end 158.077 91.573) (width 0.3) (layer F.Cu) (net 1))
 (segment (start 156.5 62.3) (end 155.95 61.75) (width 0.3) (layer F.Cu) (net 1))
 (segment (start 156.5 67.3) (end 156.5 62.3) (width 0.3) (layer F.Cu) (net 1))
 (segment (start 158.4 69.2) (end 156.5 67.3) (width 0.3) (layer F.Cu) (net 1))
 (segment (start 153.66 76.96) (end 158.12 76.96) (width 0.3) (layer B.Cu) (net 1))
 (segment (start 158.12 76.96) (end 159.3875 75.6925) (width 0.3) (layer B.Cu) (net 1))
 (segment (start 159.3875 78.9025) (end 159.3875 75.6925) (width 0.3) (layer B.Cu) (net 1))
 (segment (start 159.3875 75.6925) (end 159.3875 70.1875) (width 0.3) (layer B.Cu) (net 1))
 (segment (start 159.3875 70.1875) (end 158.4 69.2) (width 0.3) (layer B.Cu) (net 1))
 (via (at 158.4 69.2) (size 0.6) (drill 0.4) (layers F.Cu B.Cu) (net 1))
 (segment (start 148.1075 97.5925) (end 148.1075 99.6325) (width 0.25) (layer B.Cu) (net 15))
 (segment (start 148.1075 99.6325) (end 148.1675 99.6925) (width 0.25) (layer B.Cu) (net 15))
 (segment (start 148.81 89.83) (end 148.04 89.83) (width 0.3) (layer B.Cu) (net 6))
 (segment (start 147.39 86.61) (end 143.4 82.62) (width 0.3) (layer B.Cu) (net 6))
 (segment (start 147.39 89.18) (end 147.39 86.61) (width 0.3) (layer B.Cu) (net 6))
 (segment (start 148.04 89.83) (end 147.39 89.18) (width 0.3) (layer B.Cu) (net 6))
 (segment (start 144.67 93.63) (end 145.13 93.63) (width 0.3) (layer F.Cu) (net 6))
 (segment (start 145.45 92.7204) (end 144.0389 91.3093) (width 0.3) (layer F.Cu) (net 6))
 (segment (start 145.45 93.31) (end 145.45 92.7204) (width 0.3) (layer F.Cu) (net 6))
 (segment (start 145.13 93.63) (end 145.45 93.31) (width 0.3) (layer F.Cu) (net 6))
 (segment (start 143.4 87.69) (end 143.4 92.36) (width 0.3) (layer B.Cu) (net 6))
 (segment (start 143.4 92.36) (end 144.67 93.63) (width 0.3) (layer B.Cu) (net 6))
 (via (at 144.67 93.63) (size 0.6) (drill 0.4) (layers F.Cu B.Cu) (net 6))
 (segment (start 143.4 82.62) (end 143.4 87.69) (width 0.3) (layer B.Cu) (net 6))
 (segment (start 143.25 71.025) (end 143.25 78.44) (width 0.3) (layer B.Cu) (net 6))
 (segment (start 144.95 69.325) (end 143.25 71.025) (width 0.3) (layer B.Cu) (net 6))
 (segment (start 145.875 68.4) (end 144.95 69.325) (width 0.3) (layer F.Cu) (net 6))
 (via (at 144.95 69.325) (size 0.6) (drill 0.4) (layers F.Cu B.Cu) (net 6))
 (segment (start 149.675 68.4) (end 145.875 68.4) (width 0.3) (layer F.Cu) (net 6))
 (segment (start 143.73 82.29) (end 143.4 82.62) (width 0.3) (layer B.Cu) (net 6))
 (segment (start 143.73 78.92) (end 143.73 82.29) (width 0.3) (layer B.Cu) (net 6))
 (segment (start 143.25 78.44) (end 143.73 78.92) (width 0.3) (layer B.Cu) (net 6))
 (segment (start 145.91 94.87) (end 147.14 94.87) (width 0.3) (layer F.Cu) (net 6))
 (segment (start 144.67 93.63) (end 145.91 94.87) (width 0.3) (layer F.Cu) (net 6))
 (segment (start 148.81 89.83) (end 148.81 90.015) (width 0.3) (layer B.Cu) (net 6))
 (segment (start 147.14 94.87) (end 146.31 94.87) (width 0.3) (layer F.Cu) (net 6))
 (segment (start 146.31 94.87) (end 145.33 95.85) (width 0.3) (layer F.Cu) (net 6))
 (segment (start 143.52 99.36) (end 143.52 101.86) (width 0.3) (layer F.Cu) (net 6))
 (segment (start 145.33 97.55) (end 143.52 99.36) (width 0.3) (layer F.Cu) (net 6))
 (segment (start 145.33 95.85) (end 145.33 97.55) (width 0.3) (layer F.Cu) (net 6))
 (segment (start 146.95 94.68) (end 147.14 94.87) (width 0.3) (layer F.Cu) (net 6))
 (segment (start 148.48 64.43) (end 150 64.43) (width 0.3) (layer B.Cu) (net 6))
 (segment (start 150.9 65.44) (end 150.9 65.35) (width 0.3) (layer F.Cu) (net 6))
 (segment (start 150.93 65.41) (end 150.9 65.44) (width 0.3) (layer F.Cu) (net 6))
 (segment (start 150.93 65.35) (end 150.93 65.41) (width 0.3) (layer F.Cu) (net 6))
 (segment (start 151.6 64.68) (end 150.93 65.35) (width 0.3) (layer F.Cu) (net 6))
 (via (at 151.6 64.68) (size 0.6) (drill 0.4) (layers F.Cu B.Cu) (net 6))
 (segment (start 151.58 64.66) (end 151.6 64.68) (width 0.3) (layer B.Cu) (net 6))
 (segment (start 151.58 63.98) (end 151.58 64.66) (width 0.3) (layer B.Cu) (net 6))
 (segment (start 151.3 63.7) (end 151.58 63.98) (width 0.3) (layer B.Cu) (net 6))
 (segment (start 150.73 63.7) (end 151.3 63.7) (width 0.3) (layer B.Cu) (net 6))
 (segment (start 150 64.43) (end 150.73 63.7) (width 0.3) (layer B.Cu) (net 6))
 (segment (start 149.675 65.775) (end 149.675 65.675) (width 0.3) (layer F.Cu) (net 6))
 (segment (start 149.675 65.675) (end 150 65.35) (width 0.3) (layer F.Cu) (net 6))
 (segment (start 150 65.35) (end 150 65.2) (width 0.3) (layer F.Cu) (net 6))
 (segment (start 150 65.2) (end 149.675 64.875) (width 0.3) (layer F.Cu) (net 6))
 (segment (start 151.9 65.35) (end 150.9 65.35) (width 0.3) (layer F.Cu) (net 6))
 (segment (start 150.9 65.35) (end 150 65.35) (width 0.3) (layer F.Cu) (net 6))
 (segment (start 150 65.35) (end 149.675 65.35) (width 0.3) (layer F.Cu) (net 6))
 (segment (start 149.675 62.1) (end 149.675 64.875) (width 0.3) (layer F.Cu) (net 6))
 (segment (start 149.675 64.875) (end 149.675 65.35) (width 0.3) (layer F.Cu) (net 6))
 (segment (start 149.675 65.35) (end 149.675 65.775) (width 0.3) (layer F.Cu) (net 6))
 (segment (start 149.675 65.775) (end 149.675 68.4) (width 0.3) (layer F.Cu) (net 6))
 (segment (start 154.575 63.75) (end 153.5 63.75) (width 0.3) (layer F.Cu) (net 6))
 (segment (start 153.5 63.75) (end 151.9 65.35) (width 0.3) (layer F.Cu) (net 6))
 (segment (start 154.575 65.375) (end 154.575 63.75) (width 0.3) (layer F.Cu) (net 6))
 (segment (start 146.4204 99.726) (end 146.4204 100.6504) (width 0.25) (layer B.Cu) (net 12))
 (segment (start 148.16 100.97) (end 149.68 102.49) (width 0.25) (layer B.Cu) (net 12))
 (segment (start 146.74 100.97) (end 148.16 100.97) (width 0.25) (layer B.Cu) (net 12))
 (segment (start 146.4204 100.6504) (end 146.74 100.97) (width 0.25) (layer B.Cu) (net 12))
 (segment (start 153.9075 99.5425) (end 153.9075 100.5625) (width 0.25) (layer B.Cu) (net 12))
 (segment (start 149.68 101.35) (end 149.68 102.49) (width 0.25) (layer F.Cu) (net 12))
 (segment (start 150.05 100.98) (end 149.68 101.35) (width 0.25) (layer F.Cu) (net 12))
 (segment (start 153.49 100.98) (end 150.05 100.98) (width 0.25) (layer F.Cu) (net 12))
 (segment (start 153.5 100.97) (end 153.49 100.98) (width 0.25) (layer F.Cu) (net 12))
 (via (at 153.5 100.97) (size 0.6) (drill 0.4) (layers F.Cu B.Cu) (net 12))
 (segment (start 153.9075 100.5625) (end 153.5 100.97) (width 0.25) (layer B.Cu) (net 12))
 (segment (start 153.7975 97.5825) (end 153.7975 99.4325) (width 0.25) (layer B.Cu) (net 12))
 (segment (start 153.7975 99.4325) (end 153.9075 99.5425) (width 0.25) (layer B.Cu) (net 12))
 (segment (start 151.12 76.96) (end 151.12 77.74) (width 0.25) (layer F.Cu) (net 10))
 (segment (start 151.12 77.74) (end 151.94 78.56) (width 0.25) (layer F.Cu) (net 10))
 (segment (start 151.94 78.56) (end 154.87 78.56) (width 0.25) (layer F.Cu) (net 10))
 (segment (start 154.87 78.56) (end 156.205 77.225) (width 0.25) (layer F.Cu) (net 10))
 (segment (start 156.205 77.225) (end 157.95 77.225) (width 0.25) (layer F.Cu) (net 10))
 (segment (start 148.58 76.96) (end 148.58 78.07) (width 0.25) (layer F.Cu) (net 5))
 (segment (start 148.58 78.07) (end 149.7416 79.2316) (width 0.25) (layer F.Cu) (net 5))
 (segment (start 149.7416 79.2316) (end 157.95 79.2316) (width 0.25) (layer F.Cu) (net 5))
 (segment (start 143.95 81.289) (end 145.591 81.289) (width 0.25) (layer F.Cu) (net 9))
 (segment (start 145.591 81.289) (end 146.41 80.47) (width 0.25) (layer F.Cu) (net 9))
 (segment (start 146.41 80.47) (end 146.41 75.74) (width 0.25) (layer F.Cu) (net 9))
 (segment (start 146.41 75.74) (end 147.21 74.94) (width 0.25) (layer F.Cu) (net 9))
 (segment (start 147.21 74.94) (end 158.66 74.94) (width 0.25) (layer F.Cu) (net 9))
 (segment (start 158.66 74.94) (end 159.425 74.175) (width 0.25) (layer F.Cu) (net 9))
 (segment (start 154.575 68.35) (end 154.575 67.275) (width 0.25) (layer F.Cu) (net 9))
 (segment (start 159.425 74.175) (end 159.425 70.45) (width 0.25) (layer F.Cu) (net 9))
 (segment (start 159.425 70.45) (end 159.1 70.125) (width 0.25) (layer F.Cu) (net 9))
 (segment (start 159.1 70.125) (end 156.35 70.125) (width 0.25) (layer F.Cu) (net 9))
 (segment (start 156.35 70.125) (end 154.575 68.35) (width 0.25) (layer F.Cu) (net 9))
 (segment (start 157.8316 89.51) (end 158.0262 89.3154) (width 0.25) (layer F.Cu) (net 2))
 (segment (start 153.88 64.43) (end 152.77 64.43) (width 0.25) (layer B.Cu) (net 4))
 (segment (start 155.4518 81.2382) (end 157.9754 81.2382) (width 0.25) (layer F.Cu) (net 4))
 (segment (start 155.16 81.53) (end 155.4518 81.2382) (width 0.25) (layer F.Cu) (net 4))
 (segment (start 155.16 83.48) (end 155.16 81.53) (width 0.25) (layer F.Cu) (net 4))
 (segment (start 154.54 84.1) (end 155.16 83.48) (width 0.25) (layer F.Cu) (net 4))
 (segment (start 150.88 84.1) (end 154.54 84.1) (width 0.25) (layer F.Cu) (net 4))
 (via (at 150.88 84.1) (size 0.6) (drill 0.4) (layers F.Cu B.Cu) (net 4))
 (segment (start 148.97 84.1) (end 150.88 84.1) (width 0.25) (layer B.Cu) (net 4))
 (segment (start 146.43 81.56) (end 148.97 84.1) (width 0.25) (layer B.Cu) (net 4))
 (segment (start 146.43 75.91) (end 146.43 81.56) (width 0.25) (layer B.Cu) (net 4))
 (segment (start 147.18 75.16) (end 146.43 75.91) (width 0.25) (layer B.Cu) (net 4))
 (segment (start 158.4 75.16) (end 147.18 75.16) (width 0.25) (layer B.Cu) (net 4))
 (segment (start 158.77 74.79) (end 158.4 75.16) (width 0.25) (layer B.Cu) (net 4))
 (segment (start 158.77 70.59) (end 158.77 74.79) (width 0.25) (layer B.Cu) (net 4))
 (segment (start 158.42 70.24) (end 158.77 70.59) (width 0.25) (layer B.Cu) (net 4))
 (segment (start 152.36 70.24) (end 158.42 70.24) (width 0.25) (layer B.Cu) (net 4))
 (segment (start 151.27 69.15) (end 152.36 70.24) (width 0.25) (layer B.Cu) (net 4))
 (segment (start 151.27 65.93) (end 151.27 69.15) (width 0.25) (layer B.Cu) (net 4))
 (segment (start 152.77 64.43) (end 151.27 65.93) (width 0.25) (layer B.Cu) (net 4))
 (segment (start 153.88 64.43) (end 156.05 64.43) (width 0.25) (layer B.Cu) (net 4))
 (segment (start 157.11 63.37) (end 157.11 62.49) (width 0.25) (layer B.Cu) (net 4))
 (segment (start 156.05 64.43) (end 157.11 63.37) (width 0.25) (layer B.Cu) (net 4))
 (segment (start 143.93 71.28) (end 143.93 78.24) (width 0.25) (layer B.Cu) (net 3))
 (segment (start 146.78 68.43) (end 143.93 71.28) (width 0.25) (layer B.Cu) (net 3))
 (via (at 149.09 85.22) (size 0.6) (drill 0.4) (layers F.Cu B.Cu) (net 3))
 (segment (start 149.09 85.22) (end 149.1214 85.2514) (width 0.25) (layer F.Cu) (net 3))
 (segment (start 148.48 68.43) (end 146.78 68.43) (width 0.25) (layer B.Cu) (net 3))
 (segment (start 149.1214 85.2514) (end 157.9754 85.2514) (width 0.25) (layer F.Cu) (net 3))
 (segment (start 144.37 80.5) (end 149.09 85.22) (width 0.25) (layer B.Cu) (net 3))
 (segment (start 144.37 78.68) (end 144.37 80.5) (width 0.25) (layer B.Cu) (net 3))
 (segment (start 143.93 78.24) (end 144.37 78.68) (width 0.25) (layer B.Cu) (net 3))
 (segment (start 144.3653 87.2453) (end 143.9627 87.2453) (width 0.25) (layer F.Cu) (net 7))
 (segment (start 144.2953 87.2453) (end 143.9627 87.2453) (width 0.25) (layer F.Cu) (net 7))
 (segment (start 147.375 62.1) (end 147.375 62.8) (width 0.3) (layer F.Cu) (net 13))
 (segment (start 144.775 60.375) (end 146.325 60.375) (width 0.3) (layer F.Cu) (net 13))
 (segment (start 146.325 60.375) (end 147.3 59.4) (width 0.3) (layer F.Cu) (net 13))
 (segment (start 147.3 59.4) (end 147.3 62.025) (width 0.3) (layer F.Cu) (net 13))
 (segment (start 147.3 62.025) (end 147.375 62.1) (width 0.3) (layer F.Cu) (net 13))
 (segment (start 146.4204 97.694) (end 146.4204 97.2996) (width 0.25) (layer B.Cu) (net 16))
 (segment (start 149.015 96.5) (end 150.1075 97.5925) (width 0.25) (layer B.Cu) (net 16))
 (segment (start 147.22 96.5) (end 149.015 96.5) (width 0.25) (layer B.Cu) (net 16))
 (segment (start 146.4204 97.2996) (end 147.22 96.5) (width 0.25) (layer B.Cu) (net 16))
 (segment (start 150.1075 97.5925) (end 151.8875 97.5925) (width 0.25) (layer B.Cu) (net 16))
 (segment (start 151.8875 97.5925) (end 151.8975 97.5825) (width 0.25) (layer B.Cu) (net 16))
 (segment (start 150.1175 97.5825) (end 150.1075 97.5925) (width 0.25) (layer B.Cu) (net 16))
 (segment (start 151.8975 97.5825) (end 151.8975 99.5325) (width 0.25) (layer B.Cu) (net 16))
 (segment (start 151.8975 99.5325) (end 151.9075 99.5425) (width 0.25) (layer B.Cu) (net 16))
 (segment (start 150.71 89.83) (end 150.71 87.8) (width 0.25) (layer B.Cu) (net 17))
 (segment (start 170.31 87.16) (end 170.325 87.175) (width 0.25) (layer B.Cu) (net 17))
 (segment (start 147.14 102.49) (end 146.09 102.49) (width 0.25) (layer B.Cu) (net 11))
 (segment (start 145.0996 101.4996) (end 145.0996 99.726) (width 0.25) (layer B.Cu) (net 11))
 (segment (start 146.09 102.49) (end 145.0996 101.4996) (width 0.25) (layer B.Cu) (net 11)))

